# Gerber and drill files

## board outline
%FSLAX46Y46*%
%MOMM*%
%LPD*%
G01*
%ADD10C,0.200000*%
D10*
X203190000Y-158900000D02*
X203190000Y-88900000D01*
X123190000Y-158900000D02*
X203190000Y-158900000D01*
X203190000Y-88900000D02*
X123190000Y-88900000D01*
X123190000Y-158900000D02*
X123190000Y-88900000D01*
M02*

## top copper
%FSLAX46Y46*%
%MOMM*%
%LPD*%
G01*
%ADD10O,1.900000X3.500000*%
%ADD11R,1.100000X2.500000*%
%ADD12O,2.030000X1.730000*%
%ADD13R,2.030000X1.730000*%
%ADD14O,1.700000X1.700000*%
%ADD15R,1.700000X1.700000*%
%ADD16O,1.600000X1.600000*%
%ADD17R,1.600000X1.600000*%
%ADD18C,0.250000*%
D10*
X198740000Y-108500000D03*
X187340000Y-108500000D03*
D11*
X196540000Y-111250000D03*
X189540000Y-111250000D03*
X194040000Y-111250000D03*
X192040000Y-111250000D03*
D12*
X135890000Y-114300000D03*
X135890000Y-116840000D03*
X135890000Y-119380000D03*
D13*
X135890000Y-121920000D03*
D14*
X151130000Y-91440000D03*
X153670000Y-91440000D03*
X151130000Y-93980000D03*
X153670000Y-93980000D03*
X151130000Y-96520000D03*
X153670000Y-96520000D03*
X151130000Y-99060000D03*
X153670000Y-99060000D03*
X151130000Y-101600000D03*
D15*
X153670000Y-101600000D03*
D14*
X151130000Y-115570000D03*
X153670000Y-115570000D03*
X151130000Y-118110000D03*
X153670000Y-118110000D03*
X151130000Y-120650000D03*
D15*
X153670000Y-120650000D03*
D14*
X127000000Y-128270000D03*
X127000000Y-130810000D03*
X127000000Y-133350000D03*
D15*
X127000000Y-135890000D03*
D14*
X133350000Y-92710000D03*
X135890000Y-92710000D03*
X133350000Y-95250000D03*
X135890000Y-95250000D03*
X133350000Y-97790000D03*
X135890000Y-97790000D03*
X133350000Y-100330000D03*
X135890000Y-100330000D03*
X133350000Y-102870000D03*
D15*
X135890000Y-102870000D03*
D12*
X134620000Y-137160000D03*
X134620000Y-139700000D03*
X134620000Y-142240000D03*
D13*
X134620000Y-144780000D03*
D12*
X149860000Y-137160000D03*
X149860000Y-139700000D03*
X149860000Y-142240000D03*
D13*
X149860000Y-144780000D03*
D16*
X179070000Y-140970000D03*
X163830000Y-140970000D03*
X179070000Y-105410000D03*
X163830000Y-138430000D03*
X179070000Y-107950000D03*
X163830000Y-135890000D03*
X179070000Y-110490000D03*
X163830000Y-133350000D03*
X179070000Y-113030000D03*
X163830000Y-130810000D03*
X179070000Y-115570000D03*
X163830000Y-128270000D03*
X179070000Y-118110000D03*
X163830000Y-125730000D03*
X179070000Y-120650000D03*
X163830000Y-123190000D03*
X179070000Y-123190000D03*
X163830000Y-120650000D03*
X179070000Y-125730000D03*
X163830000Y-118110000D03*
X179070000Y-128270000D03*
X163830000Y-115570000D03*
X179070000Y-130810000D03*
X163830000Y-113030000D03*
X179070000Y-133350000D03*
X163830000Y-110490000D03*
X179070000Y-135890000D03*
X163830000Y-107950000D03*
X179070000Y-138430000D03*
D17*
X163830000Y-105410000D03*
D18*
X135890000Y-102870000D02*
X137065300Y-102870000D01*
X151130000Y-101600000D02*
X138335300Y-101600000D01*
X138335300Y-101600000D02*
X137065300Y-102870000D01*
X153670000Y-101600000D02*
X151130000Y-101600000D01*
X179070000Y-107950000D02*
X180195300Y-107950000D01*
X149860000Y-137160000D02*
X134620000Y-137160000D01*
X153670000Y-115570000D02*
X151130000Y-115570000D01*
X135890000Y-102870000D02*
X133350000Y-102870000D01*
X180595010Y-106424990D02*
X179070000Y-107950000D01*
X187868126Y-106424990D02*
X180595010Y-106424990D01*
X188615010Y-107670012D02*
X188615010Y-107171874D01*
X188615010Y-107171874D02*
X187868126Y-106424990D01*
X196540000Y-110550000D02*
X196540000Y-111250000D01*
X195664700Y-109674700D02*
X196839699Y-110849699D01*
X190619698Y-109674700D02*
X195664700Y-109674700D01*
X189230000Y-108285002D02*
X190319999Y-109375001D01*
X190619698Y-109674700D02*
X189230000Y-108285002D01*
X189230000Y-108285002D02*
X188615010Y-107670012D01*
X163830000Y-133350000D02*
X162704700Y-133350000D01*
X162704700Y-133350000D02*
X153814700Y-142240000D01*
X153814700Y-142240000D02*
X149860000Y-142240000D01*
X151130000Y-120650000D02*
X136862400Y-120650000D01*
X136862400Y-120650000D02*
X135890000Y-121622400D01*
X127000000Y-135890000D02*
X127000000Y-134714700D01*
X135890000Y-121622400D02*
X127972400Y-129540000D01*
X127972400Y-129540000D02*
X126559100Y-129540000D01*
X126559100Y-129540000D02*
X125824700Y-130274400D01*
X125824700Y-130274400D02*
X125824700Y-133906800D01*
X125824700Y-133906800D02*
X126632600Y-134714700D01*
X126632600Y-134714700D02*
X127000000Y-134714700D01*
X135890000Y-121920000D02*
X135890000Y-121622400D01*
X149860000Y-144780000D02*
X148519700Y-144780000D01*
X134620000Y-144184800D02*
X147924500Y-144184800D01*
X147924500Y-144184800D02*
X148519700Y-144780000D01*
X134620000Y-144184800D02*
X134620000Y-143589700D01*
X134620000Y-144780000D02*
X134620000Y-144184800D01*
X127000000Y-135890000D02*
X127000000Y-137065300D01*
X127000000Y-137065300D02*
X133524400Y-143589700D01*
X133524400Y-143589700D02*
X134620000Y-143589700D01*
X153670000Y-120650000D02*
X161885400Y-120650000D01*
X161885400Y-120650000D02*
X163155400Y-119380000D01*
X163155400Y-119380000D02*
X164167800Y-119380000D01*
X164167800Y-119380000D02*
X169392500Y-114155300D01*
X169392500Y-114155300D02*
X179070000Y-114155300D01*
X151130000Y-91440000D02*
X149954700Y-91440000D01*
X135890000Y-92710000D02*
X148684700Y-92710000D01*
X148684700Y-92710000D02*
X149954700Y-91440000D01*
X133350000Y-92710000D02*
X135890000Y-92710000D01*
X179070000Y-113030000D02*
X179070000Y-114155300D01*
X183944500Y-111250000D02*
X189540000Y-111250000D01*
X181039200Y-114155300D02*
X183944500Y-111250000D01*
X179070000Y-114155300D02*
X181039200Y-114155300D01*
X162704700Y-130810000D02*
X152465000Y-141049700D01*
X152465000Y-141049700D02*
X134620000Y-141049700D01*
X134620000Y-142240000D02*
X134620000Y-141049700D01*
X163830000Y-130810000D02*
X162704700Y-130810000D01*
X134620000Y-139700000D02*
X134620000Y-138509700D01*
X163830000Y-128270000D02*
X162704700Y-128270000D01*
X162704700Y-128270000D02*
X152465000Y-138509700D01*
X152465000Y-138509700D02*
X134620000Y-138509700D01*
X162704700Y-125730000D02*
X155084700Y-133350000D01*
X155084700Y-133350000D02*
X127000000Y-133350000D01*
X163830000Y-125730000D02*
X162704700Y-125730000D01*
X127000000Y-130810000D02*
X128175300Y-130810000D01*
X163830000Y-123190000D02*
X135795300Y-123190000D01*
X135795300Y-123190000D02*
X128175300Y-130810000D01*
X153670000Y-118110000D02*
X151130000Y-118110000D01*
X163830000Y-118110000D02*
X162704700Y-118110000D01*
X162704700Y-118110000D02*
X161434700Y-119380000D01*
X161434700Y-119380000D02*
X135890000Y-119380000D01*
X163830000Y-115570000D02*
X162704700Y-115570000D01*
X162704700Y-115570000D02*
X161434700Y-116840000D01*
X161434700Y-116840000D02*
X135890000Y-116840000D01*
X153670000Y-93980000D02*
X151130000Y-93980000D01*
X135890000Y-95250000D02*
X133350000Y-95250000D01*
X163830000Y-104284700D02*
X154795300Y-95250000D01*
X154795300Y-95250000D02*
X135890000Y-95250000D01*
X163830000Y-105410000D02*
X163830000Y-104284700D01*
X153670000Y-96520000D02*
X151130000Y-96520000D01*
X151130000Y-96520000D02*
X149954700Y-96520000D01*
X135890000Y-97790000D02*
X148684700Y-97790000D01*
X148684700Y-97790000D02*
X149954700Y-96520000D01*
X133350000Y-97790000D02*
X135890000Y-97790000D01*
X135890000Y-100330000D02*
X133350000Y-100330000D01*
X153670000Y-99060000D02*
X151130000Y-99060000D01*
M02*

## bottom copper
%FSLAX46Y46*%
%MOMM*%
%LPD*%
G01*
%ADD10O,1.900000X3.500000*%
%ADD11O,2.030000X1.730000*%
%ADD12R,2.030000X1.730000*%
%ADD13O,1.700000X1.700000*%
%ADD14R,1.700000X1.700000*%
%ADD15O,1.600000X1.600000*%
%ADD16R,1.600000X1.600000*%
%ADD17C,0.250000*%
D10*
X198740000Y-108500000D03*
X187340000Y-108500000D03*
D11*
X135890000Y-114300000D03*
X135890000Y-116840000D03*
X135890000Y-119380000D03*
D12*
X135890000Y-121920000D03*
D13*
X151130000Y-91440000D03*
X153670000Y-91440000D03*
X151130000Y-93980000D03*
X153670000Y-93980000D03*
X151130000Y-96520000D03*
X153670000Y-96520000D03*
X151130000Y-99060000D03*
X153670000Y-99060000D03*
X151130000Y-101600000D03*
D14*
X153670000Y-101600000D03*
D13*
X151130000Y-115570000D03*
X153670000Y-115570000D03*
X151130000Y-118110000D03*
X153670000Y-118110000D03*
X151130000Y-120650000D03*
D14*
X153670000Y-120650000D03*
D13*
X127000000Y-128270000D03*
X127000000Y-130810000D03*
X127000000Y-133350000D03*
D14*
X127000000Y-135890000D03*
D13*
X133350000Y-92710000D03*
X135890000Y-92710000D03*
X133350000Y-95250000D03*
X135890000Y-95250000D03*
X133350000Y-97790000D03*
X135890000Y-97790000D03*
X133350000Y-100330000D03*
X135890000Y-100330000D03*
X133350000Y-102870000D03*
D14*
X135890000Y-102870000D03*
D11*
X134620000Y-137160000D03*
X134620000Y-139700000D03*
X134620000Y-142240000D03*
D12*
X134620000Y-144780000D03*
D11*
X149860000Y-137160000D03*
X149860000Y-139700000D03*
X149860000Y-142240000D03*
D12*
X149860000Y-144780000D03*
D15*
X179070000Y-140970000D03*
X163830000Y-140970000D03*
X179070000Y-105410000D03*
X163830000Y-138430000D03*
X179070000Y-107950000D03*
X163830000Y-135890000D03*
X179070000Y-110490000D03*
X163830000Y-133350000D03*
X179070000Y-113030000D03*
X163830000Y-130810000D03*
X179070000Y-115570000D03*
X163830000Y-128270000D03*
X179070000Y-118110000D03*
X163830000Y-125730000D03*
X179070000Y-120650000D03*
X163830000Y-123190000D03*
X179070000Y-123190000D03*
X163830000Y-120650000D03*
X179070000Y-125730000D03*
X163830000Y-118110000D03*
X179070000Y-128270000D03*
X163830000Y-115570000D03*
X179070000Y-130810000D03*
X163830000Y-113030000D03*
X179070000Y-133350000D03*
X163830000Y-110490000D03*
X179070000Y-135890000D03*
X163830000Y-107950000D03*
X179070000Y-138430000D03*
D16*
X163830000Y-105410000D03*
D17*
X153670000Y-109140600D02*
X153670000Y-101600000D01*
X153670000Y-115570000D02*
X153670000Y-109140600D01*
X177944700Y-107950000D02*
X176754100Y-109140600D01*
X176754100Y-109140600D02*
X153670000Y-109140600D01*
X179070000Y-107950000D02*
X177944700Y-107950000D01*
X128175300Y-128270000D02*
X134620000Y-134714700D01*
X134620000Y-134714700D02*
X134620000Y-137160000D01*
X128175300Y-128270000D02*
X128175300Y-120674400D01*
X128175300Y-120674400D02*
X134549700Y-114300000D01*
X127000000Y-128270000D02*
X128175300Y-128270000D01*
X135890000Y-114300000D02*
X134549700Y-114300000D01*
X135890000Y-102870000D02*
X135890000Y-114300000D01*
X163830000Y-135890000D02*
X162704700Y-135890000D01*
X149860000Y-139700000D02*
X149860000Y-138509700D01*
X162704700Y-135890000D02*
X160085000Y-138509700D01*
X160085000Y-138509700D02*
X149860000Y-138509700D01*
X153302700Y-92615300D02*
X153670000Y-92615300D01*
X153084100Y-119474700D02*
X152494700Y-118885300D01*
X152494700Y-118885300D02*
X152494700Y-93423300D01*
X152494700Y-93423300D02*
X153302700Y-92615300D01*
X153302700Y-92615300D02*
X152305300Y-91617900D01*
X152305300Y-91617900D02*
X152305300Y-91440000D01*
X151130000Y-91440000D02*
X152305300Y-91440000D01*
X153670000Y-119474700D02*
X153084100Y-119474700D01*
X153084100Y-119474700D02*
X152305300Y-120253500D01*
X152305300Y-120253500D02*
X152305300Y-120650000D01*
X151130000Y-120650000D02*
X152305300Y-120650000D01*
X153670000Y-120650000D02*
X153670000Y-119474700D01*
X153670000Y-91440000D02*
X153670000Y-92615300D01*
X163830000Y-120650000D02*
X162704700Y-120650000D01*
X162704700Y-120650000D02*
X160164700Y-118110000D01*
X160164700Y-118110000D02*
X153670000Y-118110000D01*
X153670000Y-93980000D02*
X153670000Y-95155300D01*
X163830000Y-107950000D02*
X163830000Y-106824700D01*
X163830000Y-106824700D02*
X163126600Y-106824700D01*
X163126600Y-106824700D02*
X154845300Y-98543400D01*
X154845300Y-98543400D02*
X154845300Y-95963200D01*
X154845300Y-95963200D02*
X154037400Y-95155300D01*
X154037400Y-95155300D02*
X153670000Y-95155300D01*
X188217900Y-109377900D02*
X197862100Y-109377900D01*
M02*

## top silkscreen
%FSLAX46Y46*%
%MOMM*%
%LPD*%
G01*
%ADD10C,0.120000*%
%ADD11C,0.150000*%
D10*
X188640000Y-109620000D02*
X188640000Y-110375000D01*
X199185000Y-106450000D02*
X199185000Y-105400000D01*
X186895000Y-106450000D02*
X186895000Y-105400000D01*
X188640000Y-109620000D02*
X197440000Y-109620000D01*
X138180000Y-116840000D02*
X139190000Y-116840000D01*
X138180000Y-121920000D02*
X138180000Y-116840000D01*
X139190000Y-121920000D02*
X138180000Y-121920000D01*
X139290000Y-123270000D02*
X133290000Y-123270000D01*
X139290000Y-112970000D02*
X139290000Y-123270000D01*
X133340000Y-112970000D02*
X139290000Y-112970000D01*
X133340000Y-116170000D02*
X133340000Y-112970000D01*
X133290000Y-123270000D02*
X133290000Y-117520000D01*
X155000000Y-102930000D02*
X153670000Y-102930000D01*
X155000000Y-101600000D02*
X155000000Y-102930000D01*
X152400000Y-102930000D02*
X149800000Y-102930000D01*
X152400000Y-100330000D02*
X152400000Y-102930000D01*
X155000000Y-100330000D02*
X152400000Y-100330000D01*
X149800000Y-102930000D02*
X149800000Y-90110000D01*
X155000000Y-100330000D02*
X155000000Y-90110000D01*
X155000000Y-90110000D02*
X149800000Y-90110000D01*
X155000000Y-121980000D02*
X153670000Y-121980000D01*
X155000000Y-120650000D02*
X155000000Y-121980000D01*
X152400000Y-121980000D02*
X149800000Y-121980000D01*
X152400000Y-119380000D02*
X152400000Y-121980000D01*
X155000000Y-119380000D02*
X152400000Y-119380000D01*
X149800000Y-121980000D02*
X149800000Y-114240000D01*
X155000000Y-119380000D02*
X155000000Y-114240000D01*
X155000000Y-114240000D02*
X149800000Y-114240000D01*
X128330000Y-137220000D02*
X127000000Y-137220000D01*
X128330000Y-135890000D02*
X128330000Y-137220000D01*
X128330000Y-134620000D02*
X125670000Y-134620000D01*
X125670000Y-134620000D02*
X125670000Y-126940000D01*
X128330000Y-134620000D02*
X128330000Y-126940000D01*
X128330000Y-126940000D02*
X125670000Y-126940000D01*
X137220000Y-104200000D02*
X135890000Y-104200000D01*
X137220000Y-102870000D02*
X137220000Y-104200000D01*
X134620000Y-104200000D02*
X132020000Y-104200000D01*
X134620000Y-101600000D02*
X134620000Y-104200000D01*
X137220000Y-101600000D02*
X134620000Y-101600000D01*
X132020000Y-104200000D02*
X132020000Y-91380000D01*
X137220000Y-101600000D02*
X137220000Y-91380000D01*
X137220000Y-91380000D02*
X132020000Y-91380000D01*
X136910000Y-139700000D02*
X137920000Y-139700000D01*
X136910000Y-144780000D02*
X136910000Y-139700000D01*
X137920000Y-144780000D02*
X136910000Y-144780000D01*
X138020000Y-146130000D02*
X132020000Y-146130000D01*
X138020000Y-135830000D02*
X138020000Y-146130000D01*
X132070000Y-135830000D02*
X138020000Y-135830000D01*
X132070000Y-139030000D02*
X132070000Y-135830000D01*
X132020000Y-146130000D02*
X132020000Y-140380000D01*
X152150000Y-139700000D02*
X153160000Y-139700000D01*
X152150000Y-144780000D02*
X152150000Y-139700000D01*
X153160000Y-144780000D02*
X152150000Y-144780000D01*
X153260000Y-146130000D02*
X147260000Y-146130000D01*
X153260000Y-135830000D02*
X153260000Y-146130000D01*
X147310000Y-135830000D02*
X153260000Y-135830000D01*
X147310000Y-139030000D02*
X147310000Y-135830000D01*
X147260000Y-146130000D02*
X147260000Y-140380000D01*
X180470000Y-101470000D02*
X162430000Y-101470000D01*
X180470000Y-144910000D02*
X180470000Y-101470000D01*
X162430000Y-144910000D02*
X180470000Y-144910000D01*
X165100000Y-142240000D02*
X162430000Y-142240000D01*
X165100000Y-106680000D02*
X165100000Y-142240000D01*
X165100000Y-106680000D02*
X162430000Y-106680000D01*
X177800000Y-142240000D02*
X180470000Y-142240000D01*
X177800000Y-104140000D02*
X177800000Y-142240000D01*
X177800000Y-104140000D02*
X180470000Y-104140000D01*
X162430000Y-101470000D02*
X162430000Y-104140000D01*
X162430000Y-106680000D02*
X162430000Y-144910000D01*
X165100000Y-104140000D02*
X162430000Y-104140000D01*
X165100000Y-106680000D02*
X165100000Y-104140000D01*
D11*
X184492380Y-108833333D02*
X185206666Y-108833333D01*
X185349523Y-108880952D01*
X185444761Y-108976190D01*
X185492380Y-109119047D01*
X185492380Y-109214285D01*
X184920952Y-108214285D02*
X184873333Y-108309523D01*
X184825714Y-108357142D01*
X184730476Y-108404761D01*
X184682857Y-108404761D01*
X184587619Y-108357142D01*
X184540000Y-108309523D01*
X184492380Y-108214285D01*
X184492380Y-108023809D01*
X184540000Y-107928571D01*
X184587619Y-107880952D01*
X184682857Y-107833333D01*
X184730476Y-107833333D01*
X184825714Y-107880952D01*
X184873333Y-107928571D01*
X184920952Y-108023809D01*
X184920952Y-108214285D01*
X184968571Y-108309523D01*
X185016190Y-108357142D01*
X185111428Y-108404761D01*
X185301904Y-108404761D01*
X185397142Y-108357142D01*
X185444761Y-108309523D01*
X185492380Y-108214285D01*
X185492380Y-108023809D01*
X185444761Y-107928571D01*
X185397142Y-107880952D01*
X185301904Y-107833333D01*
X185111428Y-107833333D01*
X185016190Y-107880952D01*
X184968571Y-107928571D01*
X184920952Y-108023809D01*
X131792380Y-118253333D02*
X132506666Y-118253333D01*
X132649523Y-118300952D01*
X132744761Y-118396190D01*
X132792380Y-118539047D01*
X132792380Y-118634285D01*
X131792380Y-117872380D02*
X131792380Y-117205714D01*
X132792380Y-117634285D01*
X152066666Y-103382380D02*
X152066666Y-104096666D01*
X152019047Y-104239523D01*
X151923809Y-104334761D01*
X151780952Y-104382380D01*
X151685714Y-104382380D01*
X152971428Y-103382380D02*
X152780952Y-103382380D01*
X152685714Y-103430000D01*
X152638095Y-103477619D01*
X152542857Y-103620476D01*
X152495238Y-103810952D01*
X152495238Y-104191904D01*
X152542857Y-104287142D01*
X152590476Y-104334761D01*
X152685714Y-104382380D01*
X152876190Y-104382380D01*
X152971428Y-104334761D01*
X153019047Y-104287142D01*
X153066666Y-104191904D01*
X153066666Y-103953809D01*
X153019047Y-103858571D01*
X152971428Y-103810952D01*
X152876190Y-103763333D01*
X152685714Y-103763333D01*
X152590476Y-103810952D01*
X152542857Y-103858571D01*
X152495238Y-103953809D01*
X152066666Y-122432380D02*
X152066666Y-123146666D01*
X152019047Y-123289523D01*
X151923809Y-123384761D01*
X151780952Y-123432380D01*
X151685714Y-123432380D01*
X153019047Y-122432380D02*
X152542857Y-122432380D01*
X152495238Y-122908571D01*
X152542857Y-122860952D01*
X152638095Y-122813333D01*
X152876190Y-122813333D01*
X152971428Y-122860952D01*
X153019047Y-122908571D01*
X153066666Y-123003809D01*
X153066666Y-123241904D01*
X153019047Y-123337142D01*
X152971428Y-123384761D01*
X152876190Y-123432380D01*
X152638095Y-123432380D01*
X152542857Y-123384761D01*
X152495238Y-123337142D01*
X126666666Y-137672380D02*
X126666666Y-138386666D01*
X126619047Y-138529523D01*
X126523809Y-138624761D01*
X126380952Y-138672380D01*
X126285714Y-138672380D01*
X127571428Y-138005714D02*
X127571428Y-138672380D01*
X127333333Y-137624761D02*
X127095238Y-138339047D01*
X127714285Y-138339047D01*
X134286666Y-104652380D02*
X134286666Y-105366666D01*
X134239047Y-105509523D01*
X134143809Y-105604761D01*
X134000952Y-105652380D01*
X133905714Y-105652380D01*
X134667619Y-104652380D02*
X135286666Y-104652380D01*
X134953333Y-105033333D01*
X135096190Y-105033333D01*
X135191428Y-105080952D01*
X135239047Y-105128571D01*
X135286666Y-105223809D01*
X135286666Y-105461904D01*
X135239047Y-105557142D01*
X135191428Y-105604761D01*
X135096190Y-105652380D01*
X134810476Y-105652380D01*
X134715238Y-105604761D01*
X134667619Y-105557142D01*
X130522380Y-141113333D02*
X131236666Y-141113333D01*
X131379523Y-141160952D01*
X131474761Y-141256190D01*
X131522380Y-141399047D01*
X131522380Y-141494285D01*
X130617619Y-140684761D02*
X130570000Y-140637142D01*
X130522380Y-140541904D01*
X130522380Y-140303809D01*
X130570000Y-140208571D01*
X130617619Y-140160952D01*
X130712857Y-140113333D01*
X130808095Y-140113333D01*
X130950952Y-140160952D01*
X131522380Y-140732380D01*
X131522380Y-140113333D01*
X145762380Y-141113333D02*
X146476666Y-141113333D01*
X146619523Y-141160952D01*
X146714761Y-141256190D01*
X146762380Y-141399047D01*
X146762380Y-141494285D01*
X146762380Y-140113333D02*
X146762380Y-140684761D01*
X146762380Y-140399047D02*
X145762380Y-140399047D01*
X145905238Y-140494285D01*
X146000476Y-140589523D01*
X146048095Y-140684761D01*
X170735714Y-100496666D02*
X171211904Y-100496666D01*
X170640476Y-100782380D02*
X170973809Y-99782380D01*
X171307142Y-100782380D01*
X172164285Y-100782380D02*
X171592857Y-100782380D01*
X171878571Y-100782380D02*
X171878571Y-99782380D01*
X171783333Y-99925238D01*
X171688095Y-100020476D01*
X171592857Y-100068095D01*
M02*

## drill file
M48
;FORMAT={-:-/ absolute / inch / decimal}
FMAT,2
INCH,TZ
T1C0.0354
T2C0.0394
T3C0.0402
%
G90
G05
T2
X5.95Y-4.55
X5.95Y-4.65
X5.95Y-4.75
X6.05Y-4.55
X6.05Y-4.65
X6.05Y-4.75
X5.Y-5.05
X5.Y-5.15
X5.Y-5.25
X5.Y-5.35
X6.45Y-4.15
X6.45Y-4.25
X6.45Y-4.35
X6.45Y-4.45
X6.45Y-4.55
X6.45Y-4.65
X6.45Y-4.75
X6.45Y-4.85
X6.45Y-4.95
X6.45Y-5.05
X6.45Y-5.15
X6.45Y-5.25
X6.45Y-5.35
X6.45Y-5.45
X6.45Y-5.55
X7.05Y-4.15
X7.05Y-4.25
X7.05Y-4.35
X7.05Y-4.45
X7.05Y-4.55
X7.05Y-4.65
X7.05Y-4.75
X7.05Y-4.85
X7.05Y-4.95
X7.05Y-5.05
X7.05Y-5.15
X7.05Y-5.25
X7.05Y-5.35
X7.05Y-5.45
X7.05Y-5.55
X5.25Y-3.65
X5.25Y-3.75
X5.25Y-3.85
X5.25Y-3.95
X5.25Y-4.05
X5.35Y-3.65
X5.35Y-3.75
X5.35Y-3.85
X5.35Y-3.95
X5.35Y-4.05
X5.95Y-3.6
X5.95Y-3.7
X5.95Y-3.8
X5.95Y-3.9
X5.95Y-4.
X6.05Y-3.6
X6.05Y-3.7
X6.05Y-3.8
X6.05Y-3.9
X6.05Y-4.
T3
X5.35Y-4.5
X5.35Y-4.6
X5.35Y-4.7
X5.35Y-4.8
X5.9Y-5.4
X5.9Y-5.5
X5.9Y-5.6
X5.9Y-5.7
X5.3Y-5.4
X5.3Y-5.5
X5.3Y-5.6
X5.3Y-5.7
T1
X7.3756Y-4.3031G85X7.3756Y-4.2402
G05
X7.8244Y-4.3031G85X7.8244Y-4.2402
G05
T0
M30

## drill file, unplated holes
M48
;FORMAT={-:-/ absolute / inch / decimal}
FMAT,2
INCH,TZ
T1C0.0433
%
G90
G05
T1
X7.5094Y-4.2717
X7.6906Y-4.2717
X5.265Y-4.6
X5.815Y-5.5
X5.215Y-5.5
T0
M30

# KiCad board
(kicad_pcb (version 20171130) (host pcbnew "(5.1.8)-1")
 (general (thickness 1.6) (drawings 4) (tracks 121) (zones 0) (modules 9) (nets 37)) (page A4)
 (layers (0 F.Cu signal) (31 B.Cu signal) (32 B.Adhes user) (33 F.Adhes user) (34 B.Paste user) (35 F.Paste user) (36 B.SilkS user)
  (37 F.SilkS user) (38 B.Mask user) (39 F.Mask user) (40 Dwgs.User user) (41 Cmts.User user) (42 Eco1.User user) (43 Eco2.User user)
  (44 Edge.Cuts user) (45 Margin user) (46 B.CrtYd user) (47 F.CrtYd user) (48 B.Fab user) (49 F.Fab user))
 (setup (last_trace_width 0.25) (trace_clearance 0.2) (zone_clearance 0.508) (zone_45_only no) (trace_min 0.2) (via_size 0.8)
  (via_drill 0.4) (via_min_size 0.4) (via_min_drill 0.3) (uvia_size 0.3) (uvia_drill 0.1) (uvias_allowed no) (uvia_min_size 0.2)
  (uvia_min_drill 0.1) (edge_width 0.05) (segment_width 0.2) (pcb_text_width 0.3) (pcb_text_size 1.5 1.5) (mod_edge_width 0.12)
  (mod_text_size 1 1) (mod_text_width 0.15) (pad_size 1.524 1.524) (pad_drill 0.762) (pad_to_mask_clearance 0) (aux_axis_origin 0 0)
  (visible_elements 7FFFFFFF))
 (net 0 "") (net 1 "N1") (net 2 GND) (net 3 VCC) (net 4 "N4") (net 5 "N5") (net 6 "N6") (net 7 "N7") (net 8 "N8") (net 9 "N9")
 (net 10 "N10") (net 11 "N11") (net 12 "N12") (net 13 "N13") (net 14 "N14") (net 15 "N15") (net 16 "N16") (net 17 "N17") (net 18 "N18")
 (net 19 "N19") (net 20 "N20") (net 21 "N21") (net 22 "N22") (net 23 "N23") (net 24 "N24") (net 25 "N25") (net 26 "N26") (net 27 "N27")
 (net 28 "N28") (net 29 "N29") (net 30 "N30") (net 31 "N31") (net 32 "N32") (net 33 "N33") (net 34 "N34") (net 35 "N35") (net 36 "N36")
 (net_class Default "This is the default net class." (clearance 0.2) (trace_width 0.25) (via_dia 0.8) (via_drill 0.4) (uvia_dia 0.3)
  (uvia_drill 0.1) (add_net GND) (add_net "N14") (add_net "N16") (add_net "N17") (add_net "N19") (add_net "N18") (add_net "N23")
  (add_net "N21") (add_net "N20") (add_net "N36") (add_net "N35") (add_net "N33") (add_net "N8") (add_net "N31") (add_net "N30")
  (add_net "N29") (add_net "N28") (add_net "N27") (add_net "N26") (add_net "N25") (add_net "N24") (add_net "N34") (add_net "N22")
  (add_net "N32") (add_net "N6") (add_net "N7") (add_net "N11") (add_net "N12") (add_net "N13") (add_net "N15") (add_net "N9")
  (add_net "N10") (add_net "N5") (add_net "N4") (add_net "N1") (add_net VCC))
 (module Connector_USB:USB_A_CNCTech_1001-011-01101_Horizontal (layer F.Cu) (at 193.04 101.6 90)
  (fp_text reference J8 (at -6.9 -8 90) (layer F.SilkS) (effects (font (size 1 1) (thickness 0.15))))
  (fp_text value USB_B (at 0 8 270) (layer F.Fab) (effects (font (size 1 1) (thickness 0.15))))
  (fp_line (start -8.02 -4.4) (end -8.775 -4.4) (layer F.SilkS) (width 0.12))
  (fp_line (start -4.85 6.145) (end -3.8 6.145) (layer F.SilkS) (width 0.12))
  (fp_line (start -4.85 -6.145) (end -3.8 -6.145) (layer F.SilkS) (width 0.12))
  (fp_line (start -8.02 -4.4) (end -8.02 4.4) (layer F.SilkS) (width 0.12))
  (pad "" np_thru_hole circle (at -6.9 2.3 90) (size 1.1 1.1) (drill 1.1) (layers *.Cu *.Mask))
  (pad "" np_thru_hole circle (at -6.9 -2.3 90) (size 1.1 1.1) (drill 1.1) (layers *.Cu *.Mask))
  (pad 5 thru_hole oval (at -6.9 5.7 90) (size 3.5 1.9) (drill oval 2.5 0.9) (layers *.Cu *.Mask) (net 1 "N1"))
  (pad 5 thru_hole oval (at -6.9 -5.7 90) (size 3.5 1.9) (drill oval 2.5 0.9) (layers *.Cu *.Mask) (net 1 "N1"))
  (pad 4 smd rect (at -9.65 3.5 90) (size 2.5 1.1) (layers F.Cu F.Paste F.Mask) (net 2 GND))
  (pad 1 smd rect (at -9.65 -3.5 90) (size 2.5 1.1) (layers F.Cu F.Paste F.Mask) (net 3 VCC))
  (pad 3 smd rect (at -9.65 1 90) (size 2.5 1.1) (layers F.Cu F.Paste F.Mask) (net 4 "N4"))
  (pad 2 smd rect (at -9.65 -1 90) (size 2.5 1.1) (layers F.Cu F.Paste F.Mask) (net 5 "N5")))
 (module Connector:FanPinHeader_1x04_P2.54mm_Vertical (layer F.Cu) (at 135.89 121.92 90)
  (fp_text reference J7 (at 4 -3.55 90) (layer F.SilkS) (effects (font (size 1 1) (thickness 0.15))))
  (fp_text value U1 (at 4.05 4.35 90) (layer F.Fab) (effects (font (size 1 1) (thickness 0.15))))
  (fp_line (start 5.08 2.29) (end 5.08 3.3) (layer F.SilkS) (width 0.12))
  (fp_line (start 0 2.29) (end 5.08 2.29) (layer F.SilkS) (width 0.12))
  (fp_line (start 0 3.3) (end 0 2.29) (layer F.SilkS) (width 0.12))
  (fp_line (start -1.35 3.4) (end -1.35 -2.6) (layer F.SilkS) (width 0.12))
  (fp_line (start 8.95 3.4) (end -1.35 3.4) (layer F.SilkS) (width 0.12))
  (fp_line (start 8.95 -2.55) (end 8.95 3.4) (layer F.SilkS) (width 0.12))
  (fp_line (start 5.75 -2.55) (end 8.95 -2.55) (layer F.SilkS) (width 0.12))
  (fp_line (start -1.35 -2.6) (end 4.4 -2.6) (layer F.SilkS) (width 0.12))
  (pad "" np_thru_hole circle (at 5.08 -2.16 180) (size 1.1 1.1) (drill 1.1) (layers *.Cu *.Mask))
  (pad 4 thru_hole oval (at 7.62 0 180) (size 2.03 1.73) (drill 1.02) (layers *.Cu *.Mask) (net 2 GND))
  (pad 3 thru_hole oval (at 5.08 0 180) (size 2.03 1.73) (drill 1.02) (layers *.Cu *.Mask) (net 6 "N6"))
  (pad 2 thru_hole oval (at 2.54 0 180) (size 2.03 1.73) (drill 1.02) (layers *.Cu *.Mask) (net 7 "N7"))
  (pad 1 thru_hole rect (at 0 0 180) (size 2.03 1.73) (drill 1.02) (layers *.Cu *.Mask) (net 3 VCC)))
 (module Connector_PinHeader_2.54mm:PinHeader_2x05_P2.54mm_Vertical (layer F.Cu) (at 153.67 101.6 180)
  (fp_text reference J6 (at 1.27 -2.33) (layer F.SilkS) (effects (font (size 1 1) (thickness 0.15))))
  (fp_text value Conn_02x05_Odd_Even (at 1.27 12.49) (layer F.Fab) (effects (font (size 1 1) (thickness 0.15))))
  (fp_line (start -1.33 -1.33) (end 0 -1.33) (layer F.SilkS) (width 0.12))
  (fp_line (start -1.33 0) (end -1.33 -1.33) (layer F.SilkS) (width 0.12))
  (fp_line (start 1.27 -1.33) (end 3.87 -1.33) (layer F.SilkS) (width 0.12))
  (fp_line (start 1.27 1.27) (end 1.27 -1.33) (layer F.SilkS) (width 0.12))
  (fp_line (start -1.33 1.27) (end 1.27 1.27) (layer F.SilkS) (width 0.12))
  (fp_line (start 3.87 -1.33) (end 3.87 11.49) (layer F.SilkS) (width 0.12))
  (fp_line (start -1.33 1.27) (end -1.33 11.49) (layer F.SilkS) (width 0.12))
  (fp_line (start -1.33 11.49) (end 3.87 11.49) (layer F.SilkS) (width 0.12))
  (pad 10 thru_hole oval (at 2.54 10.16 180) (size 1.7 1.7) (drill 1) (layers *.Cu *.Mask) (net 3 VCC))
  (pad 9 thru_hole oval (at 0 10.16 180) (size 1.7 1.7) (drill 1) (layers *.Cu *.Mask) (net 3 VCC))
  (pad 8 thru_hole oval (at 2.54 7.62 180) (size 1.7 1.7) (drill 1) (layers *.Cu *.Mask) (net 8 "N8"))
  (pad 7 thru_hole oval (at 0 7.62 180) (size 1.7 1.7) (drill 1) (layers *.Cu *.Mask) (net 8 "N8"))
  (pad 6 thru_hole oval (at 2.54 5.08 180) (size 1.7 1.7) (drill 1) (layers *.Cu *.Mask) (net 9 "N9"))
  (pad 5 thru_hole oval (at 0 5.08 180) (size 1.7 1.7) (drill 1) (layers *.Cu *.Mask) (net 9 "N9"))
  (pad 4 thru_hole oval (at 2.54 2.54 180) (size 1.7 1.7) (drill 1) (layers *.Cu *.Mask) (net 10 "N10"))
  (pad 3 thru_hole oval (at 0 2.54 180) (size 1.7 1.7) (drill 1) (layers *.Cu *.Mask) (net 10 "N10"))
  (pad 2 thru_hole oval (at 2.54 0 180) (size 1.7 1.7) (drill 1) (layers *.Cu *.Mask) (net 2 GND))
  (pad 1 thru_hole rect (at 0 0 180) (size 1.7 1.7) (drill 1) (layers *.Cu *.Mask) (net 2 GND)))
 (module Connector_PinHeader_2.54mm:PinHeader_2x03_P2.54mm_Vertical (layer F.Cu) (at 153.67 120.65 180)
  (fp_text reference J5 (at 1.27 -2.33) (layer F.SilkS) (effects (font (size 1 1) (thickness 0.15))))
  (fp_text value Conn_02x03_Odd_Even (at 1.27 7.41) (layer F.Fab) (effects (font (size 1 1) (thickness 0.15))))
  (fp_line (start -1.33 -1.33) (end 0 -1.33) (layer F.SilkS) (width 0.12))
  (fp_line (start -1.33 0) (end -1.33 -1.33) (layer F.SilkS) (width 0.12))
  (fp_line (start 1.27 -1.33) (end 3.87 -1.33) (layer F.SilkS) (width 0.12))
  (fp_line (start 1.27 1.27) (end 1.27 -1.33) (layer F.SilkS) (width 0.12))
  (fp_line (start -1.33 1.27) (end 1.27 1.27) (layer F.SilkS) (width 0.12))
  (fp_line (start 3.87 -1.33) (end 3.87 6.41) (layer F.SilkS) (width 0.12))
  (fp_line (start -1.33 1.27) (end -1.33 6.41) (layer F.SilkS) (width 0.12))
  (fp_line (start -1.33 6.41) (end 3.87 6.41) (layer F.SilkS) (width 0.12))
  (pad 6 thru_hole oval (at 2.54 5.08 180) (size 1.7 1.7) (drill 1) (layers *.Cu *.Mask) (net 2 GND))
  (pad 5 thru_hole oval (at 0 5.08 180) (size 1.7 1.7) (drill 1) (layers *.Cu *.Mask) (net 2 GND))
  (pad 4 thru_hole oval (at 2.54 2.54 180) (size 1.7 1.7) (drill 1) (layers *.Cu *.Mask) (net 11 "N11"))
  (pad 3 thru_hole oval (at 0 2.54 180) (size 1.7 1.7) (drill 1) (layers *.Cu *.Mask) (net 11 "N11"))
  (pad 2 thru_hole oval (at 2.54 0 180) (size 1.7 1.7) (drill 1) (layers *.Cu *.Mask) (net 3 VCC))
  (pad 1 thru_hole rect (at 0 0 180) (size 1.7 1.7) (drill 1) (layers *.Cu *.Mask) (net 3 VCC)))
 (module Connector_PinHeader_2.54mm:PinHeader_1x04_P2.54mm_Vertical (layer F.Cu) (at 127 135.89 180)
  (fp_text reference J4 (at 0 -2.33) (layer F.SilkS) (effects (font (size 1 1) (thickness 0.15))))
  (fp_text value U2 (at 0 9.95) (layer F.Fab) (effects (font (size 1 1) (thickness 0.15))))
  (fp_line (start -1.33 -1.33) (end 0 -1.33) (layer F.SilkS) (width 0.12))
  (fp_line (start -1.33 0) (end -1.33 -1.33) (layer F.SilkS) (width 0.12))
  (fp_line (start -1.33 1.27) (end 1.33 1.27) (layer F.SilkS) (width 0.12))
  (fp_line (start 1.33 1.27) (end 1.33 8.95) (layer F.SilkS) (width 0.12))
  (fp_line (start -1.33 1.27) (end -1.33 8.95) (layer F.SilkS) (width 0.12))
  (fp_line (start -1.33 8.95) (end 1.33 8.95) (layer F.SilkS) (width 0.12))
  (pad 4 thru_hole oval (at 0 7.62 180) (size 1.7 1.7) (drill 1) (layers *.Cu *.Mask) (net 2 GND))
  (pad 3 thru_hole oval (at 0 5.08 180) (size 1.7 1.7) (drill 1) (layers *.Cu *.Mask) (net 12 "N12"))
  (pad 2 thru_hole oval (at 0 2.54 180) (size 1.7 1.7) (drill 1) (layers *.Cu *.Mask) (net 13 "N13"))
  (pad 1 thru_hole rect (at 0 0 180) (size 1.7 1.7) (drill 1) (layers *.Cu *.Mask) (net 3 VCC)))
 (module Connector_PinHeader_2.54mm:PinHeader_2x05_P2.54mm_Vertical (layer F.Cu) (at 135.89 102.87 180)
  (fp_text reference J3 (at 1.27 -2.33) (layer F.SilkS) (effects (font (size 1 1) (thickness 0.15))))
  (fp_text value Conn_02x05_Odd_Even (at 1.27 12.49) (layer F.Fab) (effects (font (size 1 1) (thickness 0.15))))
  (fp_line (start -1.33 -1.33) (end 0 -1.33) (layer F.SilkS) (width 0.12))
  (fp_line (start -1.33 0) (end -1.33 -1.33) (layer F.SilkS) (width 0.12))
  (fp_line (start 1.27 -1.33) (end 3.87 -1.33) (layer F.SilkS) (width 0.12))
  (fp_line (start 1.27 1.27) (end 1.27 -1.33) (layer F.SilkS) (width 0.12))
  (fp_line (start -1.33 1.27) (end 1.27 1.27) (layer F.SilkS) (width 0.12))
  (fp_line (start 3.87 -1.33) (end 3.87 11.49) (layer F.SilkS) (width 0.12))
  (fp_line (start -1.33 1.27) (end -1.33 11.49) (layer F.SilkS) (width 0.12))
  (fp_line (start -1.33 11.49) (end 3.87 11.49) (layer F.SilkS) (width 0.12))
  (pad 10 thru_hole oval (at 2.54 10.16 180) (size 1.7 1.7) (drill 1) (layers *.Cu *.Mask) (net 3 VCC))
  (pad 9 thru_hole oval (at 0 10.16 180) (size 1.7 1.7) (drill 1) (layers *.Cu *.Mask) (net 3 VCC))
  (pad 8 thru_hole oval (at 2.54 7.62 180) (size 1.7 1.7) (drill 1) (layers *.Cu *.Mask) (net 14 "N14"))
  (pad 7 thru_hole oval (at 0 7.62 180) (size 1.7 1.7) (drill 1) (layers *.Cu *.Mask) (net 14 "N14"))
  (pad 6 thru_hole oval (at 2.54 5.08 180) (size 1.7 1.7) (drill 1) (layers *.Cu *.Mask) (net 9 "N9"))
  (pad 5 thru_hole oval (at 0 5.08 180) (size 1.7 1.7) (drill 1) (layers *.Cu *.Mask) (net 9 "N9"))
  (pad 4 thru_hole oval (at 2.54 2.54 180) (size 1.7 1.7) (drill 1) (layers *.Cu *.Mask) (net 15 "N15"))
  (pad 3 thru_hole oval (at 0 2.54 180) (size 1.7 1.7) (drill 1) (layers *.Cu *.Mask) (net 15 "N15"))
  (pad 2 thru_hole oval (at 2.54 0 180) (size 1.7 1.7) (drill 1) (layers *.Cu *.Mask) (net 2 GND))
  (pad 1 thru_hole rect (at 0 0 180) (size 1.7 1.7) (drill 1) (layers *.Cu *.Mask) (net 2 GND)))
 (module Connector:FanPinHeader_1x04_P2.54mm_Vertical (layer F.Cu) (at 134.62 144.78 90)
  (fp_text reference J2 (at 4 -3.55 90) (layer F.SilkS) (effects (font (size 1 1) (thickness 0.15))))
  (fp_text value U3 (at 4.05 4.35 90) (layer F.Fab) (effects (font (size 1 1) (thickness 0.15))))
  (fp_line (start 5.08 2.29) (end 5.08 3.3) (layer F.SilkS) (width 0.12))
  (fp_line (start 0 2.29) (end 5.08 2.29) (layer F.SilkS) (width 0.12))
  (fp_line (start 0 3.3) (end 0 2.29) (layer F.SilkS) (width 0.12))
  (fp_line (start -1.35 3.4) (end -1.35 -2.6) (layer F.SilkS) (width 0.12))
  (fp_line (start 8.95 3.4) (end -1.35 3.4) (layer F.SilkS) (width 0.12))
  (fp_line (start 8.95 -2.55) (end 8.95 3.4) (layer F.SilkS) (width 0.12))
  (fp_line (start 5.75 -2.55) (end 8.95 -2.55) (layer F.SilkS) (width 0.12))
  (fp_line (start -1.35 -2.6) (end 4.4 -2.6) (layer F.SilkS) (width 0.12))
  (pad "" np_thru_hole circle (at 5.08 -2.16 180) (size 1.1 1.1) (drill 1.1) (layers *.Cu *.Mask))
  (pad 4 thru_hole oval (at 7.62 0 180) (size 2.03 1.73) (drill 1.02) (layers *.Cu *.Mask) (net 2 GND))
  (pad 3 thru_hole oval (at 5.08 0 180) (size 2.03 1.73) (drill 1.02) (layers *.Cu *.Mask) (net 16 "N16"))
  (pad 2 thru_hole oval (at 2.54 0 180) (size 2.03 1.73) (drill 1.02) (layers *.Cu *.Mask) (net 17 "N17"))
  (pad 1 thru_hole rect (at 0 0 180) (size 2.03 1.73) (drill 1.02) (layers *.Cu *.Mask) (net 3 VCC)))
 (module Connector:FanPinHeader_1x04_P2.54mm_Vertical (layer F.Cu) (at 149.86 144.78 90)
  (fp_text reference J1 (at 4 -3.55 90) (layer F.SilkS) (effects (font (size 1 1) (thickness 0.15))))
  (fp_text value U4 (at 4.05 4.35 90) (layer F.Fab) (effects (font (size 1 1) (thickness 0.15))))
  (fp_line (start 5.08 2.29) (end 5.08 3.3) (layer F.SilkS) (width 0.12))
  (fp_line (start 0 2.29) (end 5.08 2.29) (layer F.SilkS) (width 0.12))
  (fp_line (start 0 3.3) (end 0 2.29) (layer F.SilkS) (width 0.12))
  (fp_line (start -1.35 3.4) (end -1.35 -2.6) (layer F.SilkS) (width 0.12))
  (fp_line (start 8.95 3.4) (end -1.35 3.4) (layer F.SilkS) (width 0.12))
  (fp_line (start 8.95 -2.55) (end 8.95 3.4) (layer F.SilkS) (width 0.12))
  (fp_line (start 5.75 -2.55) (end 8.95 -2.55) (layer F.SilkS) (width 0.12))
  (fp_line (start -1.35 -2.6) (end 4.4 -2.6) (layer F.SilkS) (width 0.12))
  (pad "" np_thru_hole circle (at 5.08 -2.16 180) (size 1.1 1.1) (drill 1.1) (layers *.Cu *.Mask))
  (pad 4 thru_hole oval (at 7.62 0 180) (size 2.03 1.73) (drill 1.02) (layers *.Cu *.Mask) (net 2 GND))
  (pad 3 thru_hole oval (at 5.08 0 180) (size 2.03 1.73) (drill 1.02) (layers *.Cu *.Mask) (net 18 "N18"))
  (pad 2 thru_hole oval (at 2.54 0 180) (size 2.03 1.73) (drill 1.02) (layers *.Cu *.Mask) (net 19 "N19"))
  (pad 1 thru_hole rect (at 0 0 180) (size 2.03 1.73) (drill 1.02) (layers *.Cu *.Mask) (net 3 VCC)))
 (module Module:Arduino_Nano (layer F.Cu) (at 163.83 105.41)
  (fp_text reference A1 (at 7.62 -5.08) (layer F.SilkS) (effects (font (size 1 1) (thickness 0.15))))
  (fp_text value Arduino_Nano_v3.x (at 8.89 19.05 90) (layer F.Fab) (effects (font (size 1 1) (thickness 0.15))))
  (fp_line (start 16.64 -3.94) (end -1.4 -3.94) (layer F.SilkS) (width 0.12))
  (fp_line (start 16.64 39.5) (end 16.64 -3.94) (layer F.SilkS) (width 0.12))
  (fp_line (start -1.4 39.5) (end 16.64 39.5) (layer F.SilkS) (width 0.12))
  (fp_line (start 1.27 36.83) (end -1.4 36.83) (layer F.SilkS) (width 0.12))
  (fp_line (start 1.27 1.27) (end 1.27 36.83) (layer F.SilkS) (width 0.12))
  (fp_line (start 1.27 1.27) (end -1.4 1.27) (layer F.SilkS) (width 0.12))
  (fp_line (start 13.97 36.83) (end 16.64 36.83) (layer F.SilkS) (width 0.12))
  (fp_line (start 13.97 -1.27) (end 13.97 36.83) (layer F.SilkS) (width 0.12))
  (fp_line (start 13.97 -1.27) (end 16.64 -1.27) (layer F.SilkS) (width 0.12))
  (fp_line (start -1.4 -3.94) (end -1.4 -1.27) (layer F.SilkS) (width 0.12))
  (fp_line (start -1.4 1.27) (end -1.4 39.5) (layer F.SilkS) (width 0.12))
  (fp_line (start 1.27 -1.27) (end -1.4 -1.27) (layer F.SilkS) (width 0.12))
  (fp_line (start 1.27 1.27) (end 1.27 -1.27) (layer F.SilkS) (width 0.12))
  (pad 16 thru_hole oval (at 15.24 35.56) (size 1.6 1.6) (drill 1) (layers *.Cu *.Mask) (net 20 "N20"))
  (pad 15 thru_hole oval (at 0 35.56) (size 1.6 1.6) (drill 1) (layers *.Cu *.Mask) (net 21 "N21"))
  (pad 30 thru_hole oval (at 15.24 0) (size 1.6 1.6) (drill 1) (layers *.Cu *.Mask) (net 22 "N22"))
  (pad 14 thru_hole oval (at 0 33.02) (size 1.6 1.6) (drill 1) (layers *.Cu *.Mask) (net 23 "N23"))
  (pad 29 thru_hole oval (at 15.24 2.54) (size 1.6 1.6) (drill 1) (layers *.Cu *.Mask) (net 2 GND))
  (pad 13 thru_hole oval (at 0 30.48) (size 1.6 1.6) (drill 1) (layers *.Cu *.Mask) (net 18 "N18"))
  (pad 28 thru_hole oval (at 15.24 5.08) (size 1.6 1.6) (drill 1) (layers *.Cu *.Mask) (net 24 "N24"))
  (pad 12 thru_hole oval (at 0 27.94) (size 1.6 1.6) (drill 1) (layers *.Cu *.Mask) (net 19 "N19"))
  (pad 27 thru_hole oval (at 15.24 7.62) (size 1.6 1.6) (drill 1) (layers *.Cu *.Mask) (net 3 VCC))
  (pad 11 thru_hole oval (at 0 25.4) (size 1.6 1.6) (drill 1) (layers *.Cu *.Mask) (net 17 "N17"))
  (pad 26 thru_hole oval (at 15.24 10.16) (size 1.6 1.6) (drill 1) (layers *.Cu *.Mask) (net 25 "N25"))
  (pad 10 thru_hole oval (at 0 22.86) (size 1.6 1.6) (drill 1) (layers *.Cu *.Mask) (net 16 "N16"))
  (pad 25 thru_hole oval (at 15.24 12.7) (size 1.6 1.6) (drill 1) (layers *.Cu *.Mask) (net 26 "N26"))
  (pad 9 thru_hole oval (at 0 20.32) (size 1.6 1.6) (drill 1) (layers *.Cu *.Mask) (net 13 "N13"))
  (pad 24 thru_hole oval (at 15.24 15.24) (size 1.6 1.6) (drill 1) (layers *.Cu *.Mask) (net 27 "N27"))
  (pad 8 thru_hole oval (at 0 17.78) (size 1.6 1.6) (drill 1) (layers *.Cu *.Mask) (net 12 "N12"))
  (pad 23 thru_hole oval (at 15.24 17.78) (size 1.6 1.6) (drill 1) (layers *.Cu *.Mask) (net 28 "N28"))
  (pad 7 thru_hole oval (at 0 15.24) (size 1.6 1.6) (drill 1) (layers *.Cu *.Mask) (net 11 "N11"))
  (pad 22 thru_hole oval (at 15.24 20.32) (size 1.6 1.6) (drill 1) (layers *.Cu *.Mask) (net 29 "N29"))
  (pad 6 thru_hole oval (at 0 12.7) (size 1.6 1.6) (drill 1) (layers *.Cu *.Mask) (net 7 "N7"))
  (pad 21 thru_hole oval (at 15.24 22.86) (size 1.6 1.6) (drill 1) (layers *.Cu *.Mask) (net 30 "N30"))
  (pad 5 thru_hole oval (at 0 10.16) (size 1.6 1.6) (drill 1) (layers *.Cu *.Mask) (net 6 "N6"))
  (pad 20 thru_hole oval (at 15.24 25.4) (size 1.6 1.6) (drill 1) (layers *.Cu *.Mask) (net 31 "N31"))
  (pad 4 thru_hole oval (at 0 7.62) (size 1.6 1.6) (drill 1) (layers *.Cu *.Mask) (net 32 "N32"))
  (pad 19 thru_hole oval (at 15.24 27.94) (size 1.6 1.6) (drill 1) (layers *.Cu *.Mask) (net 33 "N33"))
  (pad 3 thru_hole oval (at 0 5.08) (size 1.6 1.6) (drill 1) (layers *.Cu *.Mask) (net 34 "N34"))
  (pad 18 thru_hole oval (at 15.24 30.48) (size 1.6 1.6) (drill 1) (layers *.Cu *.Mask) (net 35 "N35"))
  (pad 2 thru_hole oval (at 0 2.54) (size 1.6 1.6) (drill 1) (layers *.Cu *.Mask) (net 8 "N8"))
  (pad 17 thru_hole oval (at 15.24 33.02) (size 1.6 1.6) (drill 1) (layers *.Cu *.Mask) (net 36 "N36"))
  (pad 1 thru_hole rect (at 0 0) (size 1.6 1.6) (drill 1) (layers *.Cu *.Mask) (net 14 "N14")))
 (gr_line (start 203.19 158.9) (end 203.19 88.9) (layer Edge.Cuts) (width 0.2))
 (gr_line (start 123.19 158.9) (end 203.19 158.9) (layer Edge.Cuts) (width 0.2))
 (gr_line (start 203.19 88.9) (end 123.19 88.9) (layer Edge.Cuts) (width 0.2))
 (gr_line (start 123.19 158.9) (end 123.19 88.9) (layer Edge.Cuts) (width 0.2))
 (segment (start 135.89 102.87) (end 137.0653 102.87) (width 0.25) (layer F.Cu) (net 2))
 (segment (start 151.13 101.6) (end 138.3353 101.6) (width 0.25) (layer F.Cu) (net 2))
 (segment (start 138.3353 101.6) (end 137.0653 102.87) (width 0.25) (layer F.Cu) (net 2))
 (segment (start 153.67 101.6) (end 151.13 101.6) (width 0.25) (layer F.Cu) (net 2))
 (segment (start 153.67 109.1406) (end 153.67 101.6) (width 0.25) (layer B.Cu) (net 2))
 (segment (start 153.67 115.57) (end 153.67 109.1406) (width 0.25) (layer B.Cu) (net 2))
 (segment (start 177.9447 107.95) (end 176.7541 109.1406) (width 0.25) (layer B.Cu) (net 2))
 (segment (start 176.7541 109.1406) (end 153.67 109.1406) (width 0.25) (layer B.Cu) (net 2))
 (segment (start 179.07 107.95) (end 177.9447 107.95) (width 0.25) (layer B.Cu) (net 2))
 (segment (start 128.1753 128.27) (end 134.62 134.7147) (width 0.25) (layer B.Cu) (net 2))
 (segment (start 134.62 134.7147) (end 134.62 137.16) (width 0.25) (layer B.Cu) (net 2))
 (segment (start 128.1753 128.27) (end 128.1753 120.6744) (width 0.25) (layer B.Cu) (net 2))
 (segment (start 128.1753 120.6744) (end 134.5497 114.3) (width 0.25) (layer B.Cu) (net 2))
 (segment (start 127 128.27) (end 128.1753 128.27) (width 0.25) (layer B.Cu) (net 2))
 (segment (start 135.89 114.3) (end 134.5497 114.3) (width 0.25) (layer B.Cu) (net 2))
 (segment (start 135.89 102.87) (end 135.89 114.3) (width 0.25) (layer B.Cu) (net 2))
 (segment (start 179.07 107.95) (end 180.1953 107.95) (width 0.25) (layer F.Cu) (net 2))
 (segment (start 149.86 137.16) (end 134.62 137.16) (width 0.25) (layer F.Cu) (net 2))
 (segment (start 153.67 115.57) (end 151.13 115.57) (width 0.25) (layer F.Cu) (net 2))
 (segment (start 135.89 102.87) (end 133.35 102.87) (width 0.25) (layer F.Cu) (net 2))
 (segment (start 180.59501 106.42499) (end 179.07 107.95) (width 0.25) (layer F.Cu) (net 2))
 (segment (start 187.868126 106.42499) (end 180.59501 106.42499) (width 0.25) (layer F.Cu) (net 2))
 (segment (start 188.61501 107.670012) (end 188.61501 107.171874) (width 0.25) (layer F.Cu) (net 2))
 (segment (start 188.61501 107.171874) (end 187.868126 106.42499) (width 0.25) (layer F.Cu) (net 2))
 (segment (start 190.619698 109.6747) (end 188.61501 107.670012) (width 0.25) (layer F.Cu) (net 2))
 (segment (start 196.54 109.6747) (end 190.619698 109.6747) (width 0.25) (layer F.Cu) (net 2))
 (segment (start 163.83 135.89) (end 162.7047 135.89) (width 0.25) (layer B.Cu) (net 18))
 (segment (start 149.86 139.7) (end 149.86 138.5097) (width 0.25) (layer B.Cu) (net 18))
 (segment (start 162.7047 135.89) (end 160.085 138.5097) (width 0.25) (layer B.Cu) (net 18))
 (segment (start 160.085 138.5097) (end 149.86 138.5097) (width 0.25) (layer B.Cu) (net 18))
 (segment (start 163.83 133.35) (end 162.7047 133.35) (width 0.25) (layer F.Cu) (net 19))
 (segment (start 162.7047 133.35) (end 153.8147 142.24) (width 0.25) (layer F.Cu) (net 19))
 (segment (start 153.8147 142.24) (end 149.86 142.24) (width 0.25) (layer F.Cu) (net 19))
 (segment (start 151.13 120.65) (end 136.8624 120.65) (width 0.25) (layer F.Cu) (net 3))
 (segment (start 136.8624 120.65) (end 135.89 121.6224) (width 0.25) (layer F.Cu) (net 3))
 (segment (start 127 135.89) (end 127 134.7147) (width 0.25) (layer F.Cu) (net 3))
 (segment (start 135.89 121.6224) (end 127.9724 129.54) (width 0.25) (layer F.Cu) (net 3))
 (segment (start 127.9724 129.54) (end 126.5591 129.54) (width 0.25) (layer F.Cu) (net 3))
 (segment (start 126.5591 129.54) (end 125.8247 130.2744) (width 0.25) (layer F.Cu) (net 3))
 (segment (start 125.8247 130.2744) (end 125.8247 133.9068) (width 0.25) (layer F.Cu) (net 3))
 (segment (start 125.8247 133.9068) (end 126.6326 134.7147) (width 0.25) (layer F.Cu) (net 3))
 (segment (start 126.6326 134.7147) (end 127 134.7147) (width 0.25) (layer F.Cu) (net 3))
 (segment (start 135.89 121.92) (end 135.89 121.6224) (width 0.25) (layer F.Cu) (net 3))
 (segment (start 153.3027 92.6153) (end 153.67 92.6153) (width 0.25) (layer B.Cu) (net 3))
 (segment (start 153.0841 119.4747) (end 152.4947 118.8853) (width 0.25) (layer B.Cu) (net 3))
 (segment (start 152.4947 118.8853) (end 152.4947 93.4233) (width 0.25) (layer B.Cu) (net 3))
 (segment (start 152.4947 93.4233) (end 153.3027 92.6153) (width 0.25) (layer B.Cu) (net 3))
 (segment (start 153.3027 92.6153) (end 152.3053 91.6179) (width 0.25) (layer B.Cu) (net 3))
 (segment (start 152.3053 91.6179) (end 152.3053 91.44) (width 0.25) (layer B.Cu) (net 3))
 (segment (start 151.13 91.44) (end 152.3053 91.44) (width 0.25) (layer B.Cu) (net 3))
 (segment (start 153.67 119.4747) (end 153.0841 119.4747) (width 0.25) (layer B.Cu) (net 3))
 (segment (start 153.0841 119.4747) (end 152.3053 120.2535) (width 0.25) (layer B.Cu) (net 3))
 (segment (start 152.3053 120.2535) (end 152.3053 120.65) (width 0.25) (layer B.Cu) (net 3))
 (segment (start 151.13 120.65) (end 152.3053 120.65) (width 0.25) (layer B.Cu) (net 3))
 (segment (start 149.86 144.78) (end 148.5197 144.78) (width 0.25) (layer F.Cu) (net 3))
 (segment (start 134.62 144.1848) (end 147.9245 144.1848) (width 0.25) (layer F.Cu) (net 3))
 (segment (start 147.9245 144.1848) (end 148.5197 144.78) (width 0.25) (layer F.Cu) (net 3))
 (segment (start 134.62 144.1848) (end 134.62 143.5897) (width 0.25) (layer F.Cu) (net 3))
 (segment (start 134.62 144.78) (end 134.62 144.1848) (width 0.25) (layer F.Cu) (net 3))
 (segment (start 127 135.89) (end 127 137.0653) (width 0.25) (layer F.Cu) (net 3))
 (segment (start 127 137.0653) (end 133.5244 143.5897) (width 0.25) (layer F.Cu) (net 3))
 (segment (start 133.5244 143.5897) (end 134.62 143.5897) (width 0.25) (layer F.Cu) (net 3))
 (segment (start 153.67 120.65) (end 161.8854 120.65) (width 0.25) (layer F.Cu) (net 3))
 (segment (start 161.8854 120.65) (end 163.1554 119.38) (width 0.25) (layer F.Cu) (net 3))
 (segment (start 163.1554 119.38) (end 164.1678 119.38) (width 0.25) (layer F.Cu) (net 3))
 (segment (start 164.1678 119.38) (end 169.3925 114.1553) (width 0.25) (layer F.Cu) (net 3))
 (segment (start 169.3925 114.1553) (end 179.07 114.1553) (width 0.25) (layer F.Cu) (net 3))
 (segment (start 153.67 120.65) (end 153.67 119.4747) (width 0.25) (layer B.Cu) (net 3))
 (segment (start 153.67 91.44) (end 153.67 92.6153) (width 0.25) (layer B.Cu) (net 3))
 (segment (start 151.13 91.44) (end 149.9547 91.44) (width 0.25) (layer F.Cu) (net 3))
 (segment (start 135.89 92.71) (end 148.6847 92.71) (width 0.25) (layer F.Cu) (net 3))
 (segment (start 148.6847 92.71) (end 149.9547 91.44) (width 0.25) (layer F.Cu) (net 3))
 (segment (start 133.35 92.71) (end 135.89 92.71) (width 0.25) (layer F.Cu) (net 3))
 (segment (start 179.07 113.03) (end 179.07 114.1553) (width 0.25) (layer F.Cu) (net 3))
 (segment (start 183.9445 111.25) (end 189.54 111.25) (width 0.25) (layer F.Cu) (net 3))
 (segment (start 181.0392 114.1553) (end 183.9445 111.25) (width 0.25) (layer F.Cu) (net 3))
 (segment (start 179.07 114.1553) (end 181.0392 114.1553) (width 0.25) (layer F.Cu) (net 3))
 (segment (start 162.7047 130.81) (end 152.465 141.0497) (width 0.25) (layer F.Cu) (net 17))
 (segment (start 152.465 141.0497) (end 134.62 141.0497) (width 0.25) (layer F.Cu) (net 17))
 (segment (start 134.62 142.24) (end 134.62 141.0497) (width 0.25) (layer F.Cu) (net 17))
 (segment (start 163.83 130.81) (end 162.7047 130.81) (width 0.25) (layer F.Cu) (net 17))
 (segment (start 134.62 139.7) (end 134.62 138.5097) (width 0.25) (layer F.Cu) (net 16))
 (segment (start 163.83 128.27) (end 162.7047 128.27) (width 0.25) (layer F.Cu) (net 16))
 (segment (start 162.7047 128.27) (end 152.465 138.5097) (width 0.25) (layer F.Cu) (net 16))
 (segment (start 152.465 138.5097) (end 134.62 138.5097) (width 0.25) (layer F.Cu) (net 16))
 (segment (start 162.7047 125.73) (end 155.0847 133.35) (width 0.25) (layer F.Cu) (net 13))
 (segment (start 155.0847 133.35) (end 127 133.35) (width 0.25) (layer F.Cu) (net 13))
 (segment (start 163.83 125.73) (end 162.7047 125.73) (width 0.25) (layer F.Cu) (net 13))
 (segment (start 127 130.81) (end 128.1753 130.81) (width 0.25) (layer F.Cu) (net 12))
 (segment (start 163.83 123.19) (end 135.7953 123.19) (width 0.25) (layer F.Cu) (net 12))
 (segment (start 135.7953 123.19) (end 128.1753 130.81) (width 0.25) (layer F.Cu) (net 12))
 (segment (start 153.67 118.11) (end 151.13 118.11) (width 0.25) (layer F.Cu) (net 11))
 (segment (start 163.83 120.65) (end 162.7047 120.65) (width 0.25) (layer B.Cu) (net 11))
 (segment (start 162.7047 120.65) (end 160.1647 118.11) (width 0.25) (layer B.Cu) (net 11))
 (segment (start 160.1647 118.11) (end 153.67 118.11) (width 0.25) (layer B.Cu) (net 11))
 (segment (start 163.83 118.11) (end 162.7047 118.11) (width 0.25) (layer F.Cu) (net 7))
 (segment (start 162.7047 118.11) (end 161.4347 119.38) (width 0.25) (layer F.Cu) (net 7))
 (segment (start 161.4347 119.38) (end 135.89 119.38) (width 0.25) (layer F.Cu) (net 7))
 (segment (start 163.83 115.57) (end 162.7047 115.57) (width 0.25) (layer F.Cu) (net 6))
 (segment (start 162.7047 115.57) (end 161.4347 116.84) (width 0.25) (layer F.Cu) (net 6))
 (segment (start 161.4347 116.84) (end 135.89 116.84) (width 0.25) (layer F.Cu) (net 6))
 (segment (start 153.67 93.98) (end 153.67 95.1553) (width 0.25) (layer B.Cu) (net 8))
 (segment (start 163.83 107.95) (end 163.83 106.8247) (width 0.25) (layer B.Cu) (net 8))
 (segment (start 163.83 106.8247) (end 163.1266 106.8247) (width 0.25) (layer B.Cu) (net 8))
 (segment (start 163.1266 106.8247) (end 154.8453 98.5434) (width 0.25) (layer B.Cu) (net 8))
 (segment (start 154.8453 98.5434) (end 154.8453 95.9632) (width 0.25) (layer B.Cu) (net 8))
 (segment (start 154.8453 95.9632) (end 154.0374 95.1553) (width 0.25) (layer B.Cu) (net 8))
 (segment (start 154.0374 95.1553) (end 153.67 95.1553) (width 0.25) (layer B.Cu) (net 8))
 (segment (start 153.67 93.98) (end 151.13 93.98) (width 0.25) (layer F.Cu) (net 8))
 (segment (start 135.89 95.25) (end 133.35 95.25) (width 0.25) (layer F.Cu) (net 14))
 (segment (start 163.83 104.2847) (end 154.7953 95.25) (width 0.25) (layer F.Cu) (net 14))
 (segment (start 154.7953 95.25) (end 135.89 95.25) (width 0.25) (layer F.Cu) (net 14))
 (segment (start 163.83 105.41) (end 163.83 104.2847) (width 0.25) (layer F.Cu) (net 14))
 (segment (start 153.67 96.52) (end 151.13 96.52) (width 0.25) (layer F.Cu) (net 9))
 (segment (start 151.13 96.52) (end 149.9547 96.52) (width 0.25) (layer F.Cu) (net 9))
 (segment (start 135.89 97.79) (end 148.6847 97.79) (width 0.25) (layer F.Cu) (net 9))
 (segment (start 148.6847 97.79) (end 149.9547 96.52) (width 0.25) (layer F.Cu) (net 9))
 (segment (start 133.35 97.79) (end 135.89 97.79) (width 0.25) (layer F.Cu) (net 9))
 (segment (start 135.89 100.33) (end 133.35 100.33) (width 0.25) (layer F.Cu) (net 15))
 (segment (start 153.67 99.06) (end 151.13 99.06) (width 0.25) (layer F.Cu) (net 10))
 (segment (start 188.2179 109.3779) (end 197.8621 109.3779) (width 0.25) (layer B.Cu) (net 1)))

